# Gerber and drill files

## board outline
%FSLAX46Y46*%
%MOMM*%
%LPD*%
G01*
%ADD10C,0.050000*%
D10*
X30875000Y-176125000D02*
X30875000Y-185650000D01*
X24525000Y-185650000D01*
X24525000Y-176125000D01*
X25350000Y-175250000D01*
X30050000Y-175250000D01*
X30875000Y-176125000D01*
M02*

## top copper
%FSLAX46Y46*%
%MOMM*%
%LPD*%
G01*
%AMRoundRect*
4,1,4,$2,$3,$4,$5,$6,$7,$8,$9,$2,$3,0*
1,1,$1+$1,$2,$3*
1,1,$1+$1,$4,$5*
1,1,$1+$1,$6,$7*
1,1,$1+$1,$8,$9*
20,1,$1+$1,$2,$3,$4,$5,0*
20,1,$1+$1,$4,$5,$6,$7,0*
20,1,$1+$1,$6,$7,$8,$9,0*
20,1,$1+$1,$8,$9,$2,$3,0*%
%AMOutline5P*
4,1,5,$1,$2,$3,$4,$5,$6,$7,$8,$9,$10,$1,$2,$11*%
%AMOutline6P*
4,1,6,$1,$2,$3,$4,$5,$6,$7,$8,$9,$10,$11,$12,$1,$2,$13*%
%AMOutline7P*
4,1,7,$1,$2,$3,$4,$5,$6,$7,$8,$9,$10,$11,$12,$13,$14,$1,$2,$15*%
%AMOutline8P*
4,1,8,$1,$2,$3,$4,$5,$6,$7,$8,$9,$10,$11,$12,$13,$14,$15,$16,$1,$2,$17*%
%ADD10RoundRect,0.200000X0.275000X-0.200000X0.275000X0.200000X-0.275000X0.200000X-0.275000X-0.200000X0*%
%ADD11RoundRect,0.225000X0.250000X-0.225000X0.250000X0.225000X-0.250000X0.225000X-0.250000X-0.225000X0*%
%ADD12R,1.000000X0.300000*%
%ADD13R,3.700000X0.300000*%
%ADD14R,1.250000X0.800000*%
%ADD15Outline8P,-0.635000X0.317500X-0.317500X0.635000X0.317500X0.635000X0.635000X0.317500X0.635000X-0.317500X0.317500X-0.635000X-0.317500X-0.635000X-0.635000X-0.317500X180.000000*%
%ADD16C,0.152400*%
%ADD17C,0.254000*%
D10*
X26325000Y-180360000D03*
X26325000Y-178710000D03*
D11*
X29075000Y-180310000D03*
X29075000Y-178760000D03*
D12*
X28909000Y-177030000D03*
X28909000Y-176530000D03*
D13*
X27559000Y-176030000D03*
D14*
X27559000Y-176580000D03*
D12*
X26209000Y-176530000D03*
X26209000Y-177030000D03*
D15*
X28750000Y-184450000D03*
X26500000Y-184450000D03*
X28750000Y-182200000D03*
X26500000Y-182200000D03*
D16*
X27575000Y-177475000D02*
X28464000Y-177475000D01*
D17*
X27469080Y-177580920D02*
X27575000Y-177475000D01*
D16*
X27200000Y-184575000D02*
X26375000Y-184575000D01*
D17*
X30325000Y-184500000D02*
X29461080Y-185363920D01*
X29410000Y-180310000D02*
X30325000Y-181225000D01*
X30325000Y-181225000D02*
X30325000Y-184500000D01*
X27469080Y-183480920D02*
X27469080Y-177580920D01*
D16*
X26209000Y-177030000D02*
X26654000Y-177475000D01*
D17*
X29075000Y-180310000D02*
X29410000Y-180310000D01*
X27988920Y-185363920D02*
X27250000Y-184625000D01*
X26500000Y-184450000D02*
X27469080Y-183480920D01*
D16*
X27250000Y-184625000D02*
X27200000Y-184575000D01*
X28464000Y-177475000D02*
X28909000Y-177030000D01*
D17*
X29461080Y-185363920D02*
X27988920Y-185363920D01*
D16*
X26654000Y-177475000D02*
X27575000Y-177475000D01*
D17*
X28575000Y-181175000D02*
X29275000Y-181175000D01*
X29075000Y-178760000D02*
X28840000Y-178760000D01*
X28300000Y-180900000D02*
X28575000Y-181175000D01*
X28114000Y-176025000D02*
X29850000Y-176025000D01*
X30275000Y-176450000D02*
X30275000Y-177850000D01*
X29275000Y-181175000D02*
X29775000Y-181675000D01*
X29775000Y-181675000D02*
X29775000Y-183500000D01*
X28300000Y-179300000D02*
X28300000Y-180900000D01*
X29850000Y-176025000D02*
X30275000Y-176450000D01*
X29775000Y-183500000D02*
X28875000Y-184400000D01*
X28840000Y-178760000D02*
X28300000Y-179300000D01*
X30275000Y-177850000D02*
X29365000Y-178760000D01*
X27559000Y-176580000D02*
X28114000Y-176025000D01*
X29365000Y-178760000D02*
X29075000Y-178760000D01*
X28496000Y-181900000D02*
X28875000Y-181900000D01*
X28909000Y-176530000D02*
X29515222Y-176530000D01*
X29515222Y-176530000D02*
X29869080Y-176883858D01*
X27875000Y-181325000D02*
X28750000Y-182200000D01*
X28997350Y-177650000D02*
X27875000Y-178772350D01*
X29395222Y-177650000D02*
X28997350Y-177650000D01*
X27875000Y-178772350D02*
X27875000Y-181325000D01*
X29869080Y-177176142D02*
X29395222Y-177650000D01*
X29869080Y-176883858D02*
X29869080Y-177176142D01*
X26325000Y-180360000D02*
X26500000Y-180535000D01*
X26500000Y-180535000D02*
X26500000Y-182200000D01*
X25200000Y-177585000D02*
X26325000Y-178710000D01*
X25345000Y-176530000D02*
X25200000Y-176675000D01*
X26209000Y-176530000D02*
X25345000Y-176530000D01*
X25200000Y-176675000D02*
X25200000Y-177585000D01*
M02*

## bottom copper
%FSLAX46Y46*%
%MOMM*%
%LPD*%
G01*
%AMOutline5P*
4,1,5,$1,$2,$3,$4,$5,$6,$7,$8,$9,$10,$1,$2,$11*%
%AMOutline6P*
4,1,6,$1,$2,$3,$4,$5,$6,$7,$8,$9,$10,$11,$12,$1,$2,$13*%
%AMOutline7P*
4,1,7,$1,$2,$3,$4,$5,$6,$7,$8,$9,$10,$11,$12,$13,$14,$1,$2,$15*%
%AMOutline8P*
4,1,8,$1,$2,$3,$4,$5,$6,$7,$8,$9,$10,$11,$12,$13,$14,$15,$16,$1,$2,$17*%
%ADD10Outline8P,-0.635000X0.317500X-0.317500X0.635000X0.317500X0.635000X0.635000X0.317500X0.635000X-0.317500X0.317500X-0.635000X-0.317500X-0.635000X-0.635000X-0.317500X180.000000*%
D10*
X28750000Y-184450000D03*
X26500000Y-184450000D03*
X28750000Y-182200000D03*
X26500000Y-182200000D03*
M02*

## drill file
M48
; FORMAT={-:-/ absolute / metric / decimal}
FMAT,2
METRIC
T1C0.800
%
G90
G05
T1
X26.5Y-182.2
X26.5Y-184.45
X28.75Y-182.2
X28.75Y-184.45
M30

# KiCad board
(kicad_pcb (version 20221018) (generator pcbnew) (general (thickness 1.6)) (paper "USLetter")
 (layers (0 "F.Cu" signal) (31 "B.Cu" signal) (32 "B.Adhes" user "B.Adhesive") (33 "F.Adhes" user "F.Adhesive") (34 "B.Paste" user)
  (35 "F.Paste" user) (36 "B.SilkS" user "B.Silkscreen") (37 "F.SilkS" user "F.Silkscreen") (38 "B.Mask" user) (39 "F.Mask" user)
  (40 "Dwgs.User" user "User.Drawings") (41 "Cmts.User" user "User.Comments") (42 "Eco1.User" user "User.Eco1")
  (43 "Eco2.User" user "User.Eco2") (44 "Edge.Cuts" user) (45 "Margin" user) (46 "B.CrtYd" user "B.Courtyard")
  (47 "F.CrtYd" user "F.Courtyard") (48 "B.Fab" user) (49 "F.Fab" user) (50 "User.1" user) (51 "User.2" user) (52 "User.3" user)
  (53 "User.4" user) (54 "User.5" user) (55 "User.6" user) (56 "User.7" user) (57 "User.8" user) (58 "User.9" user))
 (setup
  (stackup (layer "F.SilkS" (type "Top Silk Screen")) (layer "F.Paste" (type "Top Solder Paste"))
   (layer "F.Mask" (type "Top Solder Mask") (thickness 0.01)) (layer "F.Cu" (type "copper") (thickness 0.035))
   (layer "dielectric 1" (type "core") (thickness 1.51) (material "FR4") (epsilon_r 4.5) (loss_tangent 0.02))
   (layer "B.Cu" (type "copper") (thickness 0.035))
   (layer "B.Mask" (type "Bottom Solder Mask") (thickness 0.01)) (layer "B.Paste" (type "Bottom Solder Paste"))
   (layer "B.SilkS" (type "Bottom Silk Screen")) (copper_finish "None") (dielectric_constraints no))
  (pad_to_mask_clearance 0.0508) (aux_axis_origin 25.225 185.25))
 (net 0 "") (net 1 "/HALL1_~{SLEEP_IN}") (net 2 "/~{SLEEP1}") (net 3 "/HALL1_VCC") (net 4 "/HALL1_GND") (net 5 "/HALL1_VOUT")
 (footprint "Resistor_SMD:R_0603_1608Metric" (layer "F.Cu") (at 26.325 179.535 90)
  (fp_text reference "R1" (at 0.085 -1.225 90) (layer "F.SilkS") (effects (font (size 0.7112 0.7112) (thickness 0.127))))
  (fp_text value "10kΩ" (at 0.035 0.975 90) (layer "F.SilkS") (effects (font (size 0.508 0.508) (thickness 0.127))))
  (pad "1" smd roundrect (at -0.825 0 90) (size 0.8 0.95) (layers "F.Cu" "F.Paste" "F.Mask") (roundrect_rratio 0.25)
   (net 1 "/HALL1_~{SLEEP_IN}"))
  (pad "2" smd roundrect (at 0.825 0 90) (size 0.8 0.95) (layers "F.Cu" "F.Paste" "F.Mask") (roundrect_rratio 0.25) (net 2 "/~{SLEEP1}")))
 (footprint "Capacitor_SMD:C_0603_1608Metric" (layer "F.Cu") (at 29.075 179.535 90)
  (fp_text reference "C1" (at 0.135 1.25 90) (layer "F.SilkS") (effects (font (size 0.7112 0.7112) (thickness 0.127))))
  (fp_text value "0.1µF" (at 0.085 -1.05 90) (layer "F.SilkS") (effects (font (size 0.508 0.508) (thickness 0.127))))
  (pad "1" smd roundrect (at -0.775 0 90) (size 0.9 0.95) (layers "F.Cu" "F.Paste" "F.Mask") (roundrect_rratio 0.25) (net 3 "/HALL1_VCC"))
  (pad "2" smd roundrect (at 0.775 0 90) (size 0.9 0.95) (layers "F.Cu" "F.Paste" "F.Mask") (roundrect_rratio 0.25) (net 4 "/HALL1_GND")))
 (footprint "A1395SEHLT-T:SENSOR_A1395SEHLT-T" (layer "F.Cu") (at 27.559 176.53 180)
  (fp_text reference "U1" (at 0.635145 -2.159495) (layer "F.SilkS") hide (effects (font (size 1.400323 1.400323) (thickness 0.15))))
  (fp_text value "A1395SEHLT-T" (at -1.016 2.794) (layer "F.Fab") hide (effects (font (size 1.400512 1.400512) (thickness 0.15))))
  (pad "1" smd rect (at -1.35 -0.5 180) (size 1 0.3) (layers "F.Cu" "F.Paste" "F.Mask") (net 3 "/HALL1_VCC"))
  (pad "2" smd rect (at -1.35 0 180) (size 1 0.3) (layers "F.Cu" "F.Paste" "F.Mask") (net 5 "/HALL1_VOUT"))
  (pad "3" smd rect (at 0 0.5 90) (size 0.3 3.7) (layers "F.Cu" "F.Paste" "F.Mask") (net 4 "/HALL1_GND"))
  (pad "4" smd rect (at 0 -0.05 180) (size 1.25 0.8) (layers "F.Cu" "F.Mask") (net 4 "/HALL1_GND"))
  (pad "5" smd rect (at 1.35 0 180) (size 1 0.3) (layers "F.Cu" "F.Paste" "F.Mask") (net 2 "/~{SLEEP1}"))
  (pad "6" smd rect (at 1.35 -0.5 180) (size 1 0.3) (layers "F.Cu" "F.Paste" "F.Mask") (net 3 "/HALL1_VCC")))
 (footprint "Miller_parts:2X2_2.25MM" (layer "F.Cu") (at 27.625 183.325 180)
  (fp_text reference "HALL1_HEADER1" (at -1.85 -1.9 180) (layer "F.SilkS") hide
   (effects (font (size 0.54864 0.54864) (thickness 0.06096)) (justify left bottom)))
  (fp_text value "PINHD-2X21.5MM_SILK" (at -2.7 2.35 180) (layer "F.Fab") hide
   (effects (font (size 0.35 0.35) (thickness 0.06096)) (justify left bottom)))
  (pad "P$1" thru_hole roundrect (at -1.125 -1.125 180) (size 1.27 1.27) (drill 0.8) (layers "*.Cu" "*.Mask") (roundrect_rratio 0.25)
   (chamfer_ratio 0.25) (chamfer top_left top_right bottom_left bottom_right) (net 4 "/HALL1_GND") (solder_mask_margin 0.0762))
  (pad "P$2" thru_hole roundrect (at 1.125 -1.125 180) (size 1.27 1.27) (drill 0.8) (layers "*.Cu" "*.Mask") (roundrect_rratio 0.25)
   (chamfer_ratio 0.25) (chamfer top_left top_right bottom_left bottom_right) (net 3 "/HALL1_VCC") (solder_mask_margin 0.0762))
  (pad "P$3" thru_hole roundrect (at -1.125 1.125 180) (size 1.27 1.27) (drill 0.8) (layers "*.Cu" "*.Mask") (roundrect_rratio 0.25)
   (chamfer_ratio 0.25) (chamfer top_left top_right bottom_left bottom_right) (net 5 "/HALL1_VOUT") (solder_mask_margin 0.0762))
  (pad "P$4" thru_hole roundrect (at 1.125 1.125 180) (size 1.27 1.27) (drill 0.8) (layers "*.Cu" "*.Mask") (roundrect_rratio 0.25)
   (chamfer_ratio 0.25) (chamfer top_left top_right bottom_left bottom_right) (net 1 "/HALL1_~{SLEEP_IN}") (solder_mask_margin 0.0762)))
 (gr_poly
  (pts (xy 30.875 176.125) (xy 30.875 185.65) (xy 24.525 185.65) (xy 24.525 176.125) (xy 25.35 175.25) (xy 30.05 175.25))
  (stroke (width 0.05) (type solid)) (fill none) (layer "Edge.Cuts"))
 (segment (start 27.575 177.475) (end 28.464 177.475) (width 0.1524) (layer "F.Cu") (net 3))
 (segment (start 27.46908 177.58092) (end 27.575 177.475) (width 0.254) (layer "F.Cu") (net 3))
 (segment (start 27.2 184.575) (end 26.375 184.575) (width 0.1524) (layer "F.Cu") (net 3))
 (segment (start 30.325 184.5) (end 29.46108 185.36392) (width 0.254) (layer "F.Cu") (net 3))
 (segment (start 29.41 180.31) (end 30.325 181.225) (width 0.254) (layer "F.Cu") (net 3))
 (segment (start 30.325 181.225) (end 30.325 184.5) (width 0.254) (layer "F.Cu") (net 3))
 (segment (start 27.46908 183.48092) (end 27.46908 177.58092) (width 0.254) (layer "F.Cu") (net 3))
 (segment (start 26.209 177.03) (end 26.654 177.475) (width 0.1524) (layer "F.Cu") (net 3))
 (segment (start 29.075 180.31) (end 29.41 180.31) (width 0.254) (layer "F.Cu") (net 3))
 (segment (start 27.98892 185.36392) (end 27.25 184.625) (width 0.254) (layer "F.Cu") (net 3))
 (segment (start 26.5 184.45) (end 27.46908 183.48092) (width 0.254) (layer "F.Cu") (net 3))
 (segment (start 27.25 184.625) (end 27.2 184.575) (width 0.1524) (layer "F.Cu") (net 3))
 (segment (start 28.464 177.475) (end 28.909 177.03) (width 0.1524) (layer "F.Cu") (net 3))
 (segment (start 29.46108 185.36392) (end 27.98892 185.36392) (width 0.254) (layer "F.Cu") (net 3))
 (segment (start 26.654 177.475) (end 27.575 177.475) (width 0.1524) (layer "F.Cu") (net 3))
 (segment (start 28.575 181.175) (end 29.275 181.175) (width 0.254) (layer "F.Cu") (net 4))
 (segment (start 29.075 178.76) (end 28.84 178.76) (width 0.254) (layer "F.Cu") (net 4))
 (segment (start 28.3 180.9) (end 28.575 181.175) (width 0.254) (layer "F.Cu") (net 4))
 (segment (start 28.114 176.025) (end 29.85 176.025) (width 0.254) (layer "F.Cu") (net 4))
 (segment (start 30.275 176.45) (end 30.275 177.85) (width 0.254) (layer "F.Cu") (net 4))
 (segment (start 29.275 181.175) (end 29.775 181.675) (width 0.254) (layer "F.Cu") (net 4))
 (segment (start 29.775 181.675) (end 29.775 183.5) (width 0.254) (layer "F.Cu") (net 4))
 (segment (start 28.3 179.3) (end 28.3 180.9) (width 0.254) (layer "F.Cu") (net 4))
 (segment (start 29.85 176.025) (end 30.275 176.45) (width 0.254) (layer "F.Cu") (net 4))
 (segment (start 29.775 183.5) (end 28.875 184.4) (width 0.254) (layer "F.Cu") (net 4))
 (segment (start 28.84 178.76) (end 28.3 179.3) (width 0.254) (layer "F.Cu") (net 4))
 (segment (start 30.275 177.85) (end 29.365 178.76) (width 0.254) (layer "F.Cu") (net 4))
 (segment (start 27.559 176.58) (end 28.114 176.025) (width 0.254) (layer "F.Cu") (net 4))
 (segment (start 29.365 178.76) (end 29.075 178.76) (width 0.254) (layer "F.Cu") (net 4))
 (segment (start 28.496 181.9) (end 28.875 181.9) (width 0.254) (layer "F.Cu") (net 5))
 (segment (start 28.909 176.53) (end 29.515222 176.53) (width 0.254) (layer "F.Cu") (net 5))
 (segment (start 29.515222 176.53) (end 29.86908 176.883858) (width 0.254) (layer "F.Cu") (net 5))
 (segment (start 27.875 181.325) (end 28.75 182.2) (width 0.254) (layer "F.Cu") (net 5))
 (segment (start 28.99735 177.65) (end 27.875 178.77235) (width 0.254) (layer "F.Cu") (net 5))
 (segment (start 29.395222 177.65) (end 28.99735 177.65) (width 0.254) (layer "F.Cu") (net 5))
 (segment (start 27.875 178.77235) (end 27.875 181.325) (width 0.254) (layer "F.Cu") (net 5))
 (segment (start 29.86908 177.176142) (end 29.395222 177.65) (width 0.254) (layer "F.Cu") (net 5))
 (segment (start 29.86908 176.883858) (end 29.86908 177.176142) (width 0.254) (layer "F.Cu") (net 5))
 (segment (start 26.325 180.36) (end 26.5 180.535) (width 0.254) (layer "F.Cu") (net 1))
 (segment (start 26.5 180.535) (end 26.5 182.2) (width 0.254) (layer "F.Cu") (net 1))
 (segment (start 25.2 177.585) (end 26.325 178.71) (width 0.254) (layer "F.Cu") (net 2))
 (segment (start 25.345 176.53) (end 25.2 176.675) (width 0.254) (layer "F.Cu") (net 2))
 (segment (start 26.209 176.53) (end 25.345 176.53) (width 0.254) (layer "F.Cu") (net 2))
 (segment (start 25.2 176.675) (end 25.2 177.585) (width 0.254) (layer "F.Cu") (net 2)))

